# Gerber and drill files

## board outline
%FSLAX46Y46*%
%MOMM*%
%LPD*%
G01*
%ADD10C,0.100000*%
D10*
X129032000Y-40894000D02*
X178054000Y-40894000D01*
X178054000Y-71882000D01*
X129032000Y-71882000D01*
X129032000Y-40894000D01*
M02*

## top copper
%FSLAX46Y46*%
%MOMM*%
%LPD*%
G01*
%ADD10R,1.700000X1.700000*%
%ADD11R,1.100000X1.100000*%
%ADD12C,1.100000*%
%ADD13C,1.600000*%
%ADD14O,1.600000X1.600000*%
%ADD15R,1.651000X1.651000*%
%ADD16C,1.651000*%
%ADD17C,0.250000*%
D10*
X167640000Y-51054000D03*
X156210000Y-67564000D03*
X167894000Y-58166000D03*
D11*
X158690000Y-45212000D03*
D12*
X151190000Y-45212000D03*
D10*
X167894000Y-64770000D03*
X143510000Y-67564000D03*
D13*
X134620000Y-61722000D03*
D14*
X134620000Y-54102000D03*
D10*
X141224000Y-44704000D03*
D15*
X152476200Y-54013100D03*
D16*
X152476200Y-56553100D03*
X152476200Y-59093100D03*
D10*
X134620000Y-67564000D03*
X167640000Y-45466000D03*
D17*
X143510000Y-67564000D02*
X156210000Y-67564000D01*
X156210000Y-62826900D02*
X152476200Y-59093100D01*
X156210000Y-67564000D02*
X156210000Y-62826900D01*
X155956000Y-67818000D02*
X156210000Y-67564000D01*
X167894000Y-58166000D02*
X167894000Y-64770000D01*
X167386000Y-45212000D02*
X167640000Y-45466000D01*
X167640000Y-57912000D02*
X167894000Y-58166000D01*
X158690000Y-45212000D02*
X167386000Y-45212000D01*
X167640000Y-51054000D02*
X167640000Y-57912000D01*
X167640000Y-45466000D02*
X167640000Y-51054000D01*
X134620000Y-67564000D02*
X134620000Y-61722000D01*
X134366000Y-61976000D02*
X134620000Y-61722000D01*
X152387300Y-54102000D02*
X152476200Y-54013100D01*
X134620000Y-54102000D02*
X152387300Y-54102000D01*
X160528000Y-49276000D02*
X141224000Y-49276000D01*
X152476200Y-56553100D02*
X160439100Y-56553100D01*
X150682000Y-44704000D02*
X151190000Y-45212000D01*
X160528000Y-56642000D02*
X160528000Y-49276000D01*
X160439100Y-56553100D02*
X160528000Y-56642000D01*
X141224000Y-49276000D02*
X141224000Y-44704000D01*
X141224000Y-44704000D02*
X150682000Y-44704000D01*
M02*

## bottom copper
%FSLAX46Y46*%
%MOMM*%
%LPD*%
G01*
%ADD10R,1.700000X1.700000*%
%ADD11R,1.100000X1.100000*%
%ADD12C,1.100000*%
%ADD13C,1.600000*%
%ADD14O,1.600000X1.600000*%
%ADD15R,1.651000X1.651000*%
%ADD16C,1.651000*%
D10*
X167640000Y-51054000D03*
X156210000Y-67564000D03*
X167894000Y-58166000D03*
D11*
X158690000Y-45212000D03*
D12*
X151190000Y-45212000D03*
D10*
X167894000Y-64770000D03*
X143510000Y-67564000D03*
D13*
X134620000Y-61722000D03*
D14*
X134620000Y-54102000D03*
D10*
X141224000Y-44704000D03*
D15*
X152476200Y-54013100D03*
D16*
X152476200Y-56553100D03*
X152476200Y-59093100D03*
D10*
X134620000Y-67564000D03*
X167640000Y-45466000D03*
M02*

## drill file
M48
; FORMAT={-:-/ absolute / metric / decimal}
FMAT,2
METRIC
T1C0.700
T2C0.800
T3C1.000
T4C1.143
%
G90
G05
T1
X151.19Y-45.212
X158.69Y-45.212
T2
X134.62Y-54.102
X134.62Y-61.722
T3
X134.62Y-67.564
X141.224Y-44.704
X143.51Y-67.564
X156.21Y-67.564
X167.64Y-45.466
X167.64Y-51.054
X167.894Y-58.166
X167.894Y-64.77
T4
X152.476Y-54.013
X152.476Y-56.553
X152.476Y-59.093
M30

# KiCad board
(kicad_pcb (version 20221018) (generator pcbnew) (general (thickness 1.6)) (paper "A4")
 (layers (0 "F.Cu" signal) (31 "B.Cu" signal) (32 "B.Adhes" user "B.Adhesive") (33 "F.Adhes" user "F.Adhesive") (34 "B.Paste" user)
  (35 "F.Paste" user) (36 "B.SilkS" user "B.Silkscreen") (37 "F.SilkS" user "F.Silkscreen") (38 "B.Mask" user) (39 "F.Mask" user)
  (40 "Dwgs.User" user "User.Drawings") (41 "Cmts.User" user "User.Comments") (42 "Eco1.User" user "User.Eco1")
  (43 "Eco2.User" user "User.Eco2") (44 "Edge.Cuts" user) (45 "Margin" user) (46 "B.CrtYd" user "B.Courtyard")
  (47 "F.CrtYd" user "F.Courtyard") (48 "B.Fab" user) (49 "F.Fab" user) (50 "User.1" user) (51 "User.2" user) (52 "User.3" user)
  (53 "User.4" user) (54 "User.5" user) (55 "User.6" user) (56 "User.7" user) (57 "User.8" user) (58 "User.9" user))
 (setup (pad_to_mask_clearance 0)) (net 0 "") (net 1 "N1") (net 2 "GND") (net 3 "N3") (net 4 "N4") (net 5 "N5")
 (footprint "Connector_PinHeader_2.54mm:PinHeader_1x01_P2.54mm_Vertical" (layer "F.Cu") (at 167.64 51.054)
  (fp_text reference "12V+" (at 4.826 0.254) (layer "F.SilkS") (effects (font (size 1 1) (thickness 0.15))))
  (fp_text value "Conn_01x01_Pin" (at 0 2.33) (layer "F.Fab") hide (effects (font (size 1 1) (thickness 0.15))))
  (pad "1" thru_hole rect (at 0 0) (size 1.7 1.7) (drill 1) (layers "*.Cu" "*.Mask") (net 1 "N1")))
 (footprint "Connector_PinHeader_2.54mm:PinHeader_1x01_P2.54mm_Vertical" (layer "F.Cu") (at 156.21 67.564)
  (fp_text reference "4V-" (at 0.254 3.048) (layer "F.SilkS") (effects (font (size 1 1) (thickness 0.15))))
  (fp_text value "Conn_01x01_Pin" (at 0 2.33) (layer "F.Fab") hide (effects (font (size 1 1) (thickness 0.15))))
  (pad "1" thru_hole rect (at 0 0) (size 1.7 1.7) (drill 1) (layers "*.Cu" "*.Mask") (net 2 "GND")))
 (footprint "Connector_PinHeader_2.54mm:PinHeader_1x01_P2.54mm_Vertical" (layer "F.Cu") (at 167.894 58.166)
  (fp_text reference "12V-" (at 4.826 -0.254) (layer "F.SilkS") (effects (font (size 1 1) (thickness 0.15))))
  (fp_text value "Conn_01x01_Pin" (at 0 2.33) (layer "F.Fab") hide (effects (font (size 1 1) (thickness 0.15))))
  (pad "1" thru_hole rect (at 0 0) (size 1.7 1.7) (drill 1) (layers "*.Cu" "*.Mask") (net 1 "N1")))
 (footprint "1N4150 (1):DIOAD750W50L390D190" (layer "F.Cu") (at 154.94 45.212 180)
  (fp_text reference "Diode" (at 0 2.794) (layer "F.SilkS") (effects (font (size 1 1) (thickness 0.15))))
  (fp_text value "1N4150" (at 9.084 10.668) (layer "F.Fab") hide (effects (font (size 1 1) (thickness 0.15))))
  (pad "1" thru_hole rect (at -3.75 0 180) (size 1.1 1.1) (drill 0.7) (layers "*.Cu" "*.Mask") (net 1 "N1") (solder_mask_margin 0.102))
  (pad "2" thru_hole circle (at 3.75 0 180) (size 1.1 1.1) (drill 0.7) (layers "*.Cu" "*.Mask") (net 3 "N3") (solder_mask_margin 0.102)))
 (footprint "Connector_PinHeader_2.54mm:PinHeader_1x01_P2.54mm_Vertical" (layer "F.Cu") (at 167.894 64.77)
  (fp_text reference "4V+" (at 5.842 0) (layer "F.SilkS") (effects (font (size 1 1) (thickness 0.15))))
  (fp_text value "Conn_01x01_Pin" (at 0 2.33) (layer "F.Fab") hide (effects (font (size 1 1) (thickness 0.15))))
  (pad "1" thru_hole rect (at 0 0) (size 1.7 1.7) (drill 1) (layers "*.Cu" "*.Mask") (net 1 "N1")))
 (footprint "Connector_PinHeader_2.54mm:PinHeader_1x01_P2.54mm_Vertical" (layer "F.Cu") (at 143.51 67.564)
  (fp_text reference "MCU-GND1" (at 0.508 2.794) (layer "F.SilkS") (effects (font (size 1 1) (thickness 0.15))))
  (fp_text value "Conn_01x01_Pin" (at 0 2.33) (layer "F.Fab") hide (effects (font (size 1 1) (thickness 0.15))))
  (pad "1" thru_hole rect (at 0 0) (size 1.7 1.7) (drill 1) (layers "*.Cu" "*.Mask") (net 2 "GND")))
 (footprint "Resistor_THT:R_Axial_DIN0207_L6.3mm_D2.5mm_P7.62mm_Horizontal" (layer "F.Cu") (at 134.62 61.722 90)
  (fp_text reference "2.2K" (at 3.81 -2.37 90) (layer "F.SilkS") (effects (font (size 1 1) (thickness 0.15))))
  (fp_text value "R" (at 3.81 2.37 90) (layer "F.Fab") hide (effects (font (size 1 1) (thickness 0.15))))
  (pad "1" thru_hole circle (at 0 0 90) (size 1.6 1.6) (drill 0.8) (layers "*.Cu" "*.Mask") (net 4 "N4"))
  (pad "2" thru_hole oval (at 7.62 0 90) (size 1.6 1.6) (drill 0.8) (layers "*.Cu" "*.Mask") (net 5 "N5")))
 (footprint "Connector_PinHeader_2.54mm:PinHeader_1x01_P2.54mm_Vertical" (layer "F.Cu") (at 141.224 44.704)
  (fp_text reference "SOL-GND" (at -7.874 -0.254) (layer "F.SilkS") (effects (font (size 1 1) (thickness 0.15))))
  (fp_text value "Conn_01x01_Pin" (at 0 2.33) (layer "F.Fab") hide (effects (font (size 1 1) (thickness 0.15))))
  (pad "1" thru_hole rect (at 0 0) (size 1.7 1.7) (drill 1) (layers "*.Cu" "*.Mask") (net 3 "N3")))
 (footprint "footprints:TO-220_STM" (layer "F.Cu") (at 152.4762 54.0131 -90)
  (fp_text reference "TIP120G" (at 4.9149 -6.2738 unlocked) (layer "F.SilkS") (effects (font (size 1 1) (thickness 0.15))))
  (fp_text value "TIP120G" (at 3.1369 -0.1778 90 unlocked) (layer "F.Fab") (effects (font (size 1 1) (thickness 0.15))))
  (pad "1" thru_hole rect (at 0 0 270) (size 1.651 1.651) (drill 1.143) (layers "*.Cu" "*.Mask") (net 5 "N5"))
  (pad "2" thru_hole circle (at 2.54 0 270) (size 1.651 1.651) (drill 1.143) (layers "*.Cu" "*.Mask") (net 3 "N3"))
  (pad "3" thru_hole circle (at 5.08 0 270) (size 1.651 1.651) (drill 1.143) (layers "*.Cu" "*.Mask") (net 2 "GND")))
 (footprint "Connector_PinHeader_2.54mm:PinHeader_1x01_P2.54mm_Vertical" (layer "F.Cu") (at 134.62 67.564 90)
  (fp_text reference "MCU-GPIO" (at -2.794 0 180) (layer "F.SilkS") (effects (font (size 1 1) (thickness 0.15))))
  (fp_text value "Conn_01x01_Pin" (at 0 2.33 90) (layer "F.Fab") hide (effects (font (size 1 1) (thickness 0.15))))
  (pad "1" thru_hole rect (at 0 0 90) (size 1.7 1.7) (drill 1) (layers "*.Cu" "*.Mask") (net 4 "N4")))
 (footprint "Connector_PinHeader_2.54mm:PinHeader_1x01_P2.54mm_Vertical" (layer "F.Cu") (at 167.64 45.466)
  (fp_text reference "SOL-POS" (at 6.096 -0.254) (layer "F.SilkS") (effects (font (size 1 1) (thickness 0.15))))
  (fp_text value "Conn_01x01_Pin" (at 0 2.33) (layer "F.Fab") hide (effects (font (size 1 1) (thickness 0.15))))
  (pad "1" thru_hole rect (at 0 0) (size 1.7 1.7) (drill 1) (layers "*.Cu" "*.Mask") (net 1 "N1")))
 (gr_rect (start 129.032 40.894) (end 178.054 71.882) (stroke (width 0.1) (type default)) (fill none) (layer "Edge.Cuts"))
 (segment (start 143.51 67.564) (end 156.21 67.564) (width 0.25) (layer "F.Cu") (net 2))
 (segment (start 156.21 62.8269) (end 152.4762 59.0931) (width 0.25) (layer "F.Cu") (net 2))
 (segment (start 156.21 67.564) (end 156.21 62.8269) (width 0.25) (layer "F.Cu") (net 2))
 (segment (start 155.956 67.818) (end 156.21 67.564) (width 0.25) (layer "F.Cu") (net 2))
 (segment (start 167.894 58.166) (end 167.894 64.77) (width 0.25) (layer "F.Cu") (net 1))
 (segment (start 167.386 45.212) (end 167.64 45.466) (width 0.25) (layer "F.Cu") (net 1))
 (segment (start 167.64 57.912) (end 167.894 58.166) (width 0.25) (layer "F.Cu") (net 1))
 (segment (start 158.69 45.212) (end 167.386 45.212) (width 0.25) (layer "F.Cu") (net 1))
 (segment (start 167.64 51.054) (end 167.64 57.912) (width 0.25) (layer "F.Cu") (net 1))
 (segment (start 167.64 45.466) (end 167.64 51.054) (width 0.25) (layer "F.Cu") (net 1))
 (segment (start 134.62 67.564) (end 134.62 61.722) (width 0.25) (layer "F.Cu") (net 4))
 (segment (start 134.366 61.976) (end 134.62 61.722) (width 0.25) (layer "F.Cu") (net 4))
 (segment (start 152.3873 54.102) (end 152.4762 54.0131) (width 0.25) (layer "F.Cu") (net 5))
 (segment (start 134.62 54.102) (end 152.3873 54.102) (width 0.25) (layer "F.Cu") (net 5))
 (segment (start 160.528 49.276) (end 141.224 49.276) (width 0.25) (layer "F.Cu") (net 3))
 (segment (start 152.4762 56.5531) (end 160.4391 56.5531) (width 0.25) (layer "F.Cu") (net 3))
 (segment (start 150.682 44.704) (end 151.19 45.212) (width 0.25) (layer "F.Cu") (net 3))
 (segment (start 160.528 56.642) (end 160.528 49.276) (width 0.25) (layer "F.Cu") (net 3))
 (segment (start 160.4391 56.5531) (end 160.528 56.642) (width 0.25) (layer "F.Cu") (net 3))
 (segment (start 141.224 49.276) (end 141.224 44.704) (width 0.25) (layer "F.Cu") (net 3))
 (segment (start 141.224 44.704) (end 150.682 44.704) (width 0.25) (layer "F.Cu") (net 3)))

